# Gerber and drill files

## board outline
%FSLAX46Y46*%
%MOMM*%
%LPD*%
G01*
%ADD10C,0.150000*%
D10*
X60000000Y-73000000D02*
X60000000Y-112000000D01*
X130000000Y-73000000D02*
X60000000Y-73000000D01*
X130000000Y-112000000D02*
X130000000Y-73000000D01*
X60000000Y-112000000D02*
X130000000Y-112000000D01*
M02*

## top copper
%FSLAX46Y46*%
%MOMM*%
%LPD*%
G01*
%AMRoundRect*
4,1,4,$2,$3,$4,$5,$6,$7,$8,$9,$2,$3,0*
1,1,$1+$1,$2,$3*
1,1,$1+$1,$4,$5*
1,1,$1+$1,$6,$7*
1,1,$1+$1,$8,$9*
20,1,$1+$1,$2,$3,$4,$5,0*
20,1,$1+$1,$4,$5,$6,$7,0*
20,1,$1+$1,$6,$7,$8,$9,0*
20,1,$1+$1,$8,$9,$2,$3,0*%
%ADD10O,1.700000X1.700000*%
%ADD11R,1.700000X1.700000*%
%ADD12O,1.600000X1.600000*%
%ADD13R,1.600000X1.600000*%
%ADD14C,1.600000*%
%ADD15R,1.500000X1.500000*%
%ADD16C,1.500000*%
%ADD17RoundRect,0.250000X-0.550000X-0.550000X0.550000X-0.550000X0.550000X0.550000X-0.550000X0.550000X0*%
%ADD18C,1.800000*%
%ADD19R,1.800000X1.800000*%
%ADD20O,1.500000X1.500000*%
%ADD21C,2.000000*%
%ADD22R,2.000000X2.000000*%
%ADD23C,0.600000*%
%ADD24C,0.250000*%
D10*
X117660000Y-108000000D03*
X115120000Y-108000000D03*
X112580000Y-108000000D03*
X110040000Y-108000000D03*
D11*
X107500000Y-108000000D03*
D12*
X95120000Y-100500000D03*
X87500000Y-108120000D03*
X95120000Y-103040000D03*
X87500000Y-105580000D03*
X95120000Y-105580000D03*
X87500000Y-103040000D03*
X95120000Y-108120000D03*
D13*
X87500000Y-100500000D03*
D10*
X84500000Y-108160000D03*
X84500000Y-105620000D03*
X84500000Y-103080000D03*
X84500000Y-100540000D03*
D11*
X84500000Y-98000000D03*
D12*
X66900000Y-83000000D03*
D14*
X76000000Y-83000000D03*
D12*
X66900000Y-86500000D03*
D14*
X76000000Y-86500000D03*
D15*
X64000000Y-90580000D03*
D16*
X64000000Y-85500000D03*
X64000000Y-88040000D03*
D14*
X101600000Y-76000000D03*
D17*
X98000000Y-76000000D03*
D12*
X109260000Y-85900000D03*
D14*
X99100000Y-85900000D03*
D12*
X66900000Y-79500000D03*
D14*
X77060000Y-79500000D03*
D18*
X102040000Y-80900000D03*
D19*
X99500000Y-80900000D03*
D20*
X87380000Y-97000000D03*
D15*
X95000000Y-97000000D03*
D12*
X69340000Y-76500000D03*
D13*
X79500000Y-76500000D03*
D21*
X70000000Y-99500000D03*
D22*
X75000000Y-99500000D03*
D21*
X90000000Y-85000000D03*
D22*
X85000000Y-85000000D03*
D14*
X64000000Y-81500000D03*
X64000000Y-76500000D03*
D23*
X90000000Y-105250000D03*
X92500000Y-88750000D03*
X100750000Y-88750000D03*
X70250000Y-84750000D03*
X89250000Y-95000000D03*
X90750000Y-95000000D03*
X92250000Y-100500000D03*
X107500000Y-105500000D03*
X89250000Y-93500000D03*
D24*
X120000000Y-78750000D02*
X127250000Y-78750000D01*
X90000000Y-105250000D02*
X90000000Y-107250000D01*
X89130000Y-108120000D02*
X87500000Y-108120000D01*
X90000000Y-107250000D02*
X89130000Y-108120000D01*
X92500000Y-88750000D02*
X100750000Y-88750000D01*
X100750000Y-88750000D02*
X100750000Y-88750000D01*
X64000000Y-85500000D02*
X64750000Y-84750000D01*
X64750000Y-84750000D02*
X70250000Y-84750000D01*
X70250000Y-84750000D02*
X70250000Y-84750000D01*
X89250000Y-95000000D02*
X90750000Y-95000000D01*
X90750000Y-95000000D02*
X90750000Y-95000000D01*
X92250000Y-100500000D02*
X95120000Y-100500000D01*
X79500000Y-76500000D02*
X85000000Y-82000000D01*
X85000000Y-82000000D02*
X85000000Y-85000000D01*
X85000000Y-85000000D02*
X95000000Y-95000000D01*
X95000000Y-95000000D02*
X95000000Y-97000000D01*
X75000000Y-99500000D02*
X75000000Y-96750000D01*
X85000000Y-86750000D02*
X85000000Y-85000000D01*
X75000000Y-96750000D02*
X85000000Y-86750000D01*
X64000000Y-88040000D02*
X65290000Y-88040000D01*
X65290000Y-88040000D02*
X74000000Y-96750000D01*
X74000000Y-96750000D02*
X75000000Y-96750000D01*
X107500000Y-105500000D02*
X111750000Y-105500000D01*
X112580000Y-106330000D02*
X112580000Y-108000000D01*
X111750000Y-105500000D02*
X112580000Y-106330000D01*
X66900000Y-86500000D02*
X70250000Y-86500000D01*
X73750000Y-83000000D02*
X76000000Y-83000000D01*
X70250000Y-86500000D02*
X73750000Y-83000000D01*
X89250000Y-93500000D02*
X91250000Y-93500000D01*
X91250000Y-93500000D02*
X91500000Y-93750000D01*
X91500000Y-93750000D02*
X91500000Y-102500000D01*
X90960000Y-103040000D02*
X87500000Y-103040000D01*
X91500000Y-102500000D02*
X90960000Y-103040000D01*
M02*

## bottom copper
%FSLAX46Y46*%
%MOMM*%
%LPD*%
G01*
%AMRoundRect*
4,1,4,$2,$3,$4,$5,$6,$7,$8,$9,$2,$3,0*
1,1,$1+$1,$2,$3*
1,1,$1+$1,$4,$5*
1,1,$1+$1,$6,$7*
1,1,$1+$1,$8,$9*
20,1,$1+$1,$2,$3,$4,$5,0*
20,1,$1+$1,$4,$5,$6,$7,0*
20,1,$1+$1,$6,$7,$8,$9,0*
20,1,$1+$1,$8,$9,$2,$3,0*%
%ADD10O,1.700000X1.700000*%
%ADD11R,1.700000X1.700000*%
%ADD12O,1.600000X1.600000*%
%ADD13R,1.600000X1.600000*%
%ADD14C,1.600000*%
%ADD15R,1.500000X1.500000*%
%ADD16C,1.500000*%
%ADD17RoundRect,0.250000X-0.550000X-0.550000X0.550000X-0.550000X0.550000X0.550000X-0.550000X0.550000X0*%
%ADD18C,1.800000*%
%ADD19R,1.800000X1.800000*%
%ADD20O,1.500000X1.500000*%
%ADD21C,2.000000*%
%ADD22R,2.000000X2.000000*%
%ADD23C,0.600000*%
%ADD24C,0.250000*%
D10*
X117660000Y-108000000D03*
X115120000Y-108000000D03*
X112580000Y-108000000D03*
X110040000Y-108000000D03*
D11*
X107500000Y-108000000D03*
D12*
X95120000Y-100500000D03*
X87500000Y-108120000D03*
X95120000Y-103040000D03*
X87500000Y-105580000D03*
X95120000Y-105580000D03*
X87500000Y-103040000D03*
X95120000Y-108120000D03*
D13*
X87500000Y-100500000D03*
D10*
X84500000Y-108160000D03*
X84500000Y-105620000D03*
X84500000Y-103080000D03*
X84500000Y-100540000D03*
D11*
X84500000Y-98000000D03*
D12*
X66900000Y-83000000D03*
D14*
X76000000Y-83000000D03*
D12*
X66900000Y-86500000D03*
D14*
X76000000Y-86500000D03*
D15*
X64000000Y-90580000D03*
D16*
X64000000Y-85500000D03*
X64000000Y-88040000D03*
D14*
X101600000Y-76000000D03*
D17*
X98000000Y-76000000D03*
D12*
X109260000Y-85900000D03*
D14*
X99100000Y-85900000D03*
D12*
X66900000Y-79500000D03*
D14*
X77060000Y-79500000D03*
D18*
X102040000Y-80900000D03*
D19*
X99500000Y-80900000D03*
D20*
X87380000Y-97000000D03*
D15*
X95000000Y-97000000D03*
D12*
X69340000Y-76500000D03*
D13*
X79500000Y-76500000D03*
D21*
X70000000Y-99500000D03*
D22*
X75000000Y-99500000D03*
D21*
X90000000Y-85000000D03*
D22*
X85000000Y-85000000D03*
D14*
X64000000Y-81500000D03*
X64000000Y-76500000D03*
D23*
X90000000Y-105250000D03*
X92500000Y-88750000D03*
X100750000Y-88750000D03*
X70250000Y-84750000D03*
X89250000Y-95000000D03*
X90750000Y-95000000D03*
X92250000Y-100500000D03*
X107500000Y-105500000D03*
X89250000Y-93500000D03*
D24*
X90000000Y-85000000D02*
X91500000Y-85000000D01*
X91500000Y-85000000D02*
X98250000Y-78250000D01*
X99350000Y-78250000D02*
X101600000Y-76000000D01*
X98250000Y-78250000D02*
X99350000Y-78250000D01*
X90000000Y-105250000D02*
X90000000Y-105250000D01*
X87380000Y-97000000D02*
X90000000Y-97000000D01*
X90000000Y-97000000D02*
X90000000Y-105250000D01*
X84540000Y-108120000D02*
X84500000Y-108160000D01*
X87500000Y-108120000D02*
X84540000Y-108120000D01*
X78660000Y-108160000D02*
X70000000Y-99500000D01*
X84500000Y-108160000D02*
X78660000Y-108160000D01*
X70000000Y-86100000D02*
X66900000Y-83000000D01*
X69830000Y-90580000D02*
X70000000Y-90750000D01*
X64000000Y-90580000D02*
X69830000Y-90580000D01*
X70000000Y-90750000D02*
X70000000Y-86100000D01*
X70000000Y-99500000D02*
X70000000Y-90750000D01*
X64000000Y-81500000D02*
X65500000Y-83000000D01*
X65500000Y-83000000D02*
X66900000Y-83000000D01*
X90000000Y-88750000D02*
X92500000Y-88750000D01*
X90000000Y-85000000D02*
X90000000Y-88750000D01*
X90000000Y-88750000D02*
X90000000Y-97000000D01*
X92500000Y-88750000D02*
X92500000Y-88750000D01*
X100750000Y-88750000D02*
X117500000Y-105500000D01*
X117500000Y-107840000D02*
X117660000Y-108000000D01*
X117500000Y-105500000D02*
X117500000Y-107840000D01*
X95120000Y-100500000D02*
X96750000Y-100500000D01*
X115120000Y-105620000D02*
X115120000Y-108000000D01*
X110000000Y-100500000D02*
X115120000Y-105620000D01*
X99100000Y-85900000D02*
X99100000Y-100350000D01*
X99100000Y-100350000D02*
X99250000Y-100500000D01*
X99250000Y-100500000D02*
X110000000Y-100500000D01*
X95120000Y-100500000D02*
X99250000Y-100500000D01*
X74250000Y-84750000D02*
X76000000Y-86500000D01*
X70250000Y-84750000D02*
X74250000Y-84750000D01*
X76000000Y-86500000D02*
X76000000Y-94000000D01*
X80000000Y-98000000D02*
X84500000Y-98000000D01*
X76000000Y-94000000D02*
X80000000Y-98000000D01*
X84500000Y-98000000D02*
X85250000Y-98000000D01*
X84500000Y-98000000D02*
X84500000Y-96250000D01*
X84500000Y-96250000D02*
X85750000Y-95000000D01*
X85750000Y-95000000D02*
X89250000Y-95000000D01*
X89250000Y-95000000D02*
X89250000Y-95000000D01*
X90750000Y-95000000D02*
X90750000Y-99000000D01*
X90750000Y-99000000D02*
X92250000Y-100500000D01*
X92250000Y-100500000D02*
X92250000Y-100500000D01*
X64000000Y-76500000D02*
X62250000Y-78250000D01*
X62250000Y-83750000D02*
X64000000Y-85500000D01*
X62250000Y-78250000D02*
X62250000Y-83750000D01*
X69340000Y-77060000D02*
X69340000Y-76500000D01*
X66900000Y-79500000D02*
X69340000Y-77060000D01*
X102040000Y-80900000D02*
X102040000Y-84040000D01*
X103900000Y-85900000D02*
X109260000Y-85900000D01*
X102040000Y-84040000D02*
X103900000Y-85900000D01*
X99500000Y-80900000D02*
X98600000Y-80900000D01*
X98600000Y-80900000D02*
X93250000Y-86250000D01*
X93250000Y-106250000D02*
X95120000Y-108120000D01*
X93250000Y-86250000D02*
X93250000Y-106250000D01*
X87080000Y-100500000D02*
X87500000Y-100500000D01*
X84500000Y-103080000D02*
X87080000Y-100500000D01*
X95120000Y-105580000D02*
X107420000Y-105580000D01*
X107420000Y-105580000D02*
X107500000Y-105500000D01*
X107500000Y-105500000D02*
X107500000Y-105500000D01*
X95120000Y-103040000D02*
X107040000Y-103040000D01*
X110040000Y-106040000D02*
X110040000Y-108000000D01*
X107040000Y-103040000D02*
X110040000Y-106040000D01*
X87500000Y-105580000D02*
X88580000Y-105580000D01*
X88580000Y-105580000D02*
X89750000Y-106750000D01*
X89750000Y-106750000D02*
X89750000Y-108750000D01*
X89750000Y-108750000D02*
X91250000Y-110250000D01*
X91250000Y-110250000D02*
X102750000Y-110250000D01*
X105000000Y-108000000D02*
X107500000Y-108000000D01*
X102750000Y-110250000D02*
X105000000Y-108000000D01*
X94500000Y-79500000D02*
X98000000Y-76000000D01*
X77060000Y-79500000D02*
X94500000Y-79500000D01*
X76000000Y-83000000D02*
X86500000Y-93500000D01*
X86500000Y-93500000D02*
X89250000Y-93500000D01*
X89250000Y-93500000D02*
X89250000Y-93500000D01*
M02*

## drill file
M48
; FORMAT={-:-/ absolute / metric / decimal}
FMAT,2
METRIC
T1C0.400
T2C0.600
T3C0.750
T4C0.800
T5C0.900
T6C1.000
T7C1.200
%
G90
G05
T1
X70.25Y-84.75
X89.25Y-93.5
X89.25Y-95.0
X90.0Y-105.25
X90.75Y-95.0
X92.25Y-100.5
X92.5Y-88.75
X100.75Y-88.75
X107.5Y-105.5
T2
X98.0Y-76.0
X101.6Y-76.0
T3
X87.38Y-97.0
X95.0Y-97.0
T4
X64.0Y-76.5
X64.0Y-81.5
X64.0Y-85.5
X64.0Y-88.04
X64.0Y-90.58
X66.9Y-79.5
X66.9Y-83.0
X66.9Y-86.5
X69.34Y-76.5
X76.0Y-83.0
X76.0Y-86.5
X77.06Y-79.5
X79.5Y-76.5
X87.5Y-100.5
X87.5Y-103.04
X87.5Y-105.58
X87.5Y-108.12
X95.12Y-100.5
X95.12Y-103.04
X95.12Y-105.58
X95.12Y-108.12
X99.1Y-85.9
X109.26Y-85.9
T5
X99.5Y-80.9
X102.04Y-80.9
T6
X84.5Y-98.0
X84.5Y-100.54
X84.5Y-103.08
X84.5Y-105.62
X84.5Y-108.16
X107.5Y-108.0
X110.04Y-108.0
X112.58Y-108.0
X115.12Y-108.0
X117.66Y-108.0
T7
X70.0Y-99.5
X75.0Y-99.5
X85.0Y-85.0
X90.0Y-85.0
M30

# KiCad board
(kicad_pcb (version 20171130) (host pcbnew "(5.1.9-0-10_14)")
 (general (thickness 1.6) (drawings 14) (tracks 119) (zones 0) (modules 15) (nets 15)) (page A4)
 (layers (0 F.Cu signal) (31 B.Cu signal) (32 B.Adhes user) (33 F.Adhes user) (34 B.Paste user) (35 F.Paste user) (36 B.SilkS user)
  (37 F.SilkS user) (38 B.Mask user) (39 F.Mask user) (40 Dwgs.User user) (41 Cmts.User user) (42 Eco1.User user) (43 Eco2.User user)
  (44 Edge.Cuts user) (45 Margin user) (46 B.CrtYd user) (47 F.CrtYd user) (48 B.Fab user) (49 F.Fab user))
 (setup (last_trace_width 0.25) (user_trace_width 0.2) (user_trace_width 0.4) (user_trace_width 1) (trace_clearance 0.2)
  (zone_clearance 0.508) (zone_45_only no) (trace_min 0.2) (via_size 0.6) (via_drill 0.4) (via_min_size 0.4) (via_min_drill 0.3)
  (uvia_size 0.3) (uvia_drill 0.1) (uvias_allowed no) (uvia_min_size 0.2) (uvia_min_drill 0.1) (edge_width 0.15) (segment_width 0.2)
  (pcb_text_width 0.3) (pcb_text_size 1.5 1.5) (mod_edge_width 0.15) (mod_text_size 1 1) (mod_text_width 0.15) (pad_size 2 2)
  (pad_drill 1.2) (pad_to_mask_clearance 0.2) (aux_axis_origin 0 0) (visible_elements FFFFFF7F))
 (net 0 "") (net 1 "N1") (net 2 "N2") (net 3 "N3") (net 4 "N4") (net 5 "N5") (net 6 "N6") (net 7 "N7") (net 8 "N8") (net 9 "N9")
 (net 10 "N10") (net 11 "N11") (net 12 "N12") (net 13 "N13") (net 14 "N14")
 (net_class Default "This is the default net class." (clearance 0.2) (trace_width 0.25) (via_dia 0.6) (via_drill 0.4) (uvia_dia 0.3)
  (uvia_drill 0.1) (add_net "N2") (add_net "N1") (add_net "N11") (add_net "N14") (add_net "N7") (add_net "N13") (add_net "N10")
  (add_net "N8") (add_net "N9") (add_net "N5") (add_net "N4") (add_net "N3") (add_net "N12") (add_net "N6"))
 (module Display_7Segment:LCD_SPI (layer F.Cu) (at 97.5 110 90)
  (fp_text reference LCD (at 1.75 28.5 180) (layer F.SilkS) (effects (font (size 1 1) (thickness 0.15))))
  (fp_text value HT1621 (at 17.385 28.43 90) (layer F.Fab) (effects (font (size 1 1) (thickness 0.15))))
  (pad 5 thru_hole oval (at 2 20.16 90) (size 1.7 1.7) (drill 1) (layers *.Cu *.Mask) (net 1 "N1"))
  (pad 4 thru_hole oval (at 2 17.62 90) (size 1.7 1.7) (drill 1) (layers *.Cu *.Mask) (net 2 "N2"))
  (pad 3 thru_hole oval (at 2 15.08 90) (size 1.7 1.7) (drill 1) (layers *.Cu *.Mask) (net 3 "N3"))
  (pad 2 thru_hole oval (at 2 12.54 90) (size 1.7 1.7) (drill 1) (layers *.Cu *.Mask) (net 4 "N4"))
  (pad 1 thru_hole rect (at 2 10 90) (size 1.7 1.7) (drill 1) (layers *.Cu *.Mask) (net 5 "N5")))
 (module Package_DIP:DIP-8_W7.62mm (layer F.Cu) (at 87.5 100.5)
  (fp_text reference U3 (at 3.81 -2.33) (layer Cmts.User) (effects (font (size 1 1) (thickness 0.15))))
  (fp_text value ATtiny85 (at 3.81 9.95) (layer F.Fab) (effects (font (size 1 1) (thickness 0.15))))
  (pad 8 thru_hole oval (at 7.62 0) (size 1.6 1.6) (drill 0.8) (layers *.Cu *.Mask) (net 2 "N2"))
  (pad 4 thru_hole oval (at 0 7.62) (size 1.6 1.6) (drill 0.8) (layers *.Cu *.Mask) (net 1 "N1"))
  (pad 7 thru_hole oval (at 7.62 2.54) (size 1.6 1.6) (drill 0.8) (layers *.Cu *.Mask) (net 4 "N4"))
  (pad 3 thru_hole oval (at 0 5.08) (size 1.6 1.6) (drill 0.8) (layers *.Cu *.Mask) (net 5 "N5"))
  (pad 6 thru_hole oval (at 7.62 5.08) (size 1.6 1.6) (drill 0.8) (layers *.Cu *.Mask) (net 3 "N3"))
  (pad 2 thru_hole oval (at 0 2.54) (size 1.6 1.6) (drill 0.8) (layers *.Cu *.Mask) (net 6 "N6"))
  (pad 5 thru_hole oval (at 7.62 7.62) (size 1.6 1.6) (drill 0.8) (layers *.Cu *.Mask) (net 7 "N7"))
  (pad 1 thru_hole rect (at 0 0) (size 1.6 1.6) (drill 0.8) (layers *.Cu *.Mask) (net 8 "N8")))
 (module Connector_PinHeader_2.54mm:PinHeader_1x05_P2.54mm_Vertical (layer F.Cu) (at 84.5 98)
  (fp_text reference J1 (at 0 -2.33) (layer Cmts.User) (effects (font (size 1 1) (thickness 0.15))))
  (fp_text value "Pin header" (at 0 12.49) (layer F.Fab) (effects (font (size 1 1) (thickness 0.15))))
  (pad 5 thru_hole oval (at 0 10.16) (size 1.7 1.7) (drill 1) (layers *.Cu *.Mask) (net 1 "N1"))
  (pad 4 thru_hole oval (at 0 7.62) (size 1.7 1.7) (drill 1) (layers *.Cu *.Mask) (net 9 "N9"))
  (pad 3 thru_hole oval (at 0 5.08) (size 1.7 1.7) (drill 1) (layers *.Cu *.Mask) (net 8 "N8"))
  (pad 2 thru_hole oval (at 0 2.54) (size 1.7 1.7) (drill 1) (layers *.Cu *.Mask) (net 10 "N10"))
  (pad 1 thru_hole rect (at 0 0) (size 1.7 1.7) (drill 1) (layers *.Cu *.Mask) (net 2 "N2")))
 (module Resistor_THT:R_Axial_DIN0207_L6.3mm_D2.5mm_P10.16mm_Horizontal (layer F.Cu) (at 77 83 180)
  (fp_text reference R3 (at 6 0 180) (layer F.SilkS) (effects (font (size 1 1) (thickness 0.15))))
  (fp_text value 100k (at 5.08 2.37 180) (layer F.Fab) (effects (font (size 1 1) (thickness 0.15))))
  (pad 2 thru_hole oval (at 10.1 0 180) (size 1.6 1.6) (drill 0.8) (layers *.Cu *.Mask) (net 1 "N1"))
  (pad 1 thru_hole circle (at 1 0 180) (size 1.6 1.6) (drill 0.8) (layers *.Cu *.Mask) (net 6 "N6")))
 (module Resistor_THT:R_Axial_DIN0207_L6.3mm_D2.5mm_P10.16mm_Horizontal (layer F.Cu) (at 77 86.5 180)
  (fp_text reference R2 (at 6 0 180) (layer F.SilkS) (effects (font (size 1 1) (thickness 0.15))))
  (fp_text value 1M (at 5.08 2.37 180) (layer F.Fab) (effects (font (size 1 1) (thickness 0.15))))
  (pad 2 thru_hole oval (at 10.1 0 180) (size 1.6 1.6) (drill 0.8) (layers *.Cu *.Mask) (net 6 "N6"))
  (pad 1 thru_hole circle (at 1 0 180) (size 1.6 1.6) (drill 0.8) (layers *.Cu *.Mask) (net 2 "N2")))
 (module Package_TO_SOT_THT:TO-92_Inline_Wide (layer F.Cu) (at 64 90.58 90)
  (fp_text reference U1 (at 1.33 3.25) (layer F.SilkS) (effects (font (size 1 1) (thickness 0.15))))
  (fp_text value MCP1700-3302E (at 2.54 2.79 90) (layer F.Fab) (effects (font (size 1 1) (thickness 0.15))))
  (pad 1 thru_hole rect (at 0 0 90) (size 1.5 1.5) (drill 0.8) (layers *.Cu *.Mask) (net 1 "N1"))
  (pad 3 thru_hole circle (at 5.08 0 90) (size 1.5 1.5) (drill 0.8) (layers *.Cu *.Mask) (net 2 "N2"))
  (pad 2 thru_hole circle (at 2.54 0 90) (size 1.5 1.5) (drill 0.8) (layers *.Cu *.Mask) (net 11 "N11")))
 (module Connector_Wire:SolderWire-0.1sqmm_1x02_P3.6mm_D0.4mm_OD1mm (layer F.Cu) (at 98 76)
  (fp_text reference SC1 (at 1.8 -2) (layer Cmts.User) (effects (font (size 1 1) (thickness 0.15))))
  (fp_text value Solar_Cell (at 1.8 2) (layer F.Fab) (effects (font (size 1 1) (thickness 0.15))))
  (pad 2 thru_hole circle (at 3.6 0) (size 1.6 1.6) (drill 0.6) (layers *.Cu *.Mask) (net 1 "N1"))
  (pad 1 thru_hole roundrect (at 0 0) (size 1.6 1.6) (drill 0.6) (layers *.Cu *.Mask) (roundrect_rratio 0.15625) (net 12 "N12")))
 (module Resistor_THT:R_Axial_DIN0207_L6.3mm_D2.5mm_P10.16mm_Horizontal (layer F.Cu) (at 99.1 85.9)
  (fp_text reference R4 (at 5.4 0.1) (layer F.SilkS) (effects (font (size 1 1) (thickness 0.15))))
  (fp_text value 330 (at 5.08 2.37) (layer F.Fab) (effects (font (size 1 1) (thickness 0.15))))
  (pad 2 thru_hole oval (at 10.16 0) (size 1.6 1.6) (drill 0.8) (layers *.Cu *.Mask) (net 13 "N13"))
  (pad 1 thru_hole circle (at 0 0) (size 1.6 1.6) (drill 0.8) (layers *.Cu *.Mask) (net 2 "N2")))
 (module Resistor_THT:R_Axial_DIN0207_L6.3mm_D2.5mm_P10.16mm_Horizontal (layer F.Cu) (at 77.06 79.5 180)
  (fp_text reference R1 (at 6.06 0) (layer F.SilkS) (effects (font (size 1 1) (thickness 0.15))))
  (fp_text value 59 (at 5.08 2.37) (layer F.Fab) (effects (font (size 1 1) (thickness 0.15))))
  (pad 2 thru_hole oval (at 10.16 0 180) (size 1.6 1.6) (drill 0.8) (layers *.Cu *.Mask) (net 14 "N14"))
  (pad 1 thru_hole circle (at 0 0 180) (size 1.6 1.6) (drill 0.8) (layers *.Cu *.Mask) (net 12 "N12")))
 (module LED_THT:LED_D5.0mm (layer F.Cu) (at 99.5 80.9)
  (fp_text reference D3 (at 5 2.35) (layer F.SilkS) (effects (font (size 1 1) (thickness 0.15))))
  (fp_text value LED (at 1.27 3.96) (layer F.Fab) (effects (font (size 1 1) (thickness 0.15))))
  (pad 2 thru_hole circle (at 2.54 0) (size 1.8 1.8) (drill 0.9) (layers *.Cu *.Mask) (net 13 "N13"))
  (pad 1 thru_hole rect (at 0 0) (size 1.8 1.8) (drill 0.9) (layers *.Cu *.Mask) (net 7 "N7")))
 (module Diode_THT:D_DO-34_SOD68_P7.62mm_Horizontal (layer F.Cu) (at 95 97 180)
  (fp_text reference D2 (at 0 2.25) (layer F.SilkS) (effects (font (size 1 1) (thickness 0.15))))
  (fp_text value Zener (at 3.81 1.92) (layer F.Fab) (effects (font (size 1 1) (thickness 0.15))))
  (pad 2 thru_hole oval (at 7.62 0 180) (size 1.5 1.5) (drill 0.75) (layers *.Cu *.Mask) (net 1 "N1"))
  (pad 1 thru_hole rect (at 0 0 180) (size 1.5 1.5) (drill 0.75) (layers *.Cu *.Mask) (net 11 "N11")))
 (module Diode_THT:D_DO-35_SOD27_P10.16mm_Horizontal (layer F.Cu) (at 79.5 76.5 180)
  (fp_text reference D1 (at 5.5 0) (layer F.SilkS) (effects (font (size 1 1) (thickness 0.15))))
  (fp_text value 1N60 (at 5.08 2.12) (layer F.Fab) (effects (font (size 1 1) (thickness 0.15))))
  (pad 2 thru_hole oval (at 10.16 0 180) (size 1.6 1.6) (drill 0.8) (layers *.Cu *.Mask) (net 14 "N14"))
  (pad 1 thru_hole rect (at 0 0 180) (size 1.6 1.6) (drill 0.8) (layers *.Cu *.Mask) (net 11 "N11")))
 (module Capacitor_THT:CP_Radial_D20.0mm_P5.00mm (layer F.Cu) (at 75 99.5 180)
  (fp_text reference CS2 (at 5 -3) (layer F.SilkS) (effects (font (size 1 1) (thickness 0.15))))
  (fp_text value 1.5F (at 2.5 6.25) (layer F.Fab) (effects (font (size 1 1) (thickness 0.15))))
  (pad 2 thru_hole circle (at 5 0 180) (size 2 2) (drill 1.2) (layers *.Cu *.Mask) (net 1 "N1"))
  (pad 1 thru_hole rect (at 0 0 180) (size 2 2) (drill 1.2) (layers *.Cu *.Mask) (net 11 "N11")))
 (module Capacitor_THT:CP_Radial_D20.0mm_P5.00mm (layer F.Cu) (at 85 85)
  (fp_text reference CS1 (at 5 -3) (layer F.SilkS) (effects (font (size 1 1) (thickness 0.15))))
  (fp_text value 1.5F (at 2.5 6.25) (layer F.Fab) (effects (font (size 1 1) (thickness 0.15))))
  (pad 2 thru_hole circle (at 5 0) (size 2 2) (drill 1.2) (layers *.Cu *.Mask) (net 1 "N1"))
  (pad 1 thru_hole rect (at 0 0) (size 2 2) (drill 1.2) (layers *.Cu *.Mask) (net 11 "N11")))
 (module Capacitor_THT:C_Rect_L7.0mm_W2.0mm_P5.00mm (layer F.Cu) (at 64 76.5 270)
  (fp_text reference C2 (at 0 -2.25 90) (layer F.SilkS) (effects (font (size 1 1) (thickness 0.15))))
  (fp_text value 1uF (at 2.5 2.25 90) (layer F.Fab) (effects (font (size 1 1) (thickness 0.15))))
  (pad 2 thru_hole circle (at 5 0 270) (size 1.6 1.6) (drill 0.8) (layers *.Cu *.Mask) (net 1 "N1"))
  (pad 1 thru_hole circle (at 0 0 270) (size 1.6 1.6) (drill 0.8) (layers *.Cu *.Mask) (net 2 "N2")))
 (gr_line (start 60 73) (end 60 112) (layer Edge.Cuts) (width 0.15))
 (gr_line (start 130 73) (end 60 73) (layer Edge.Cuts) (width 0.15))
 (gr_line (start 130 112) (end 130 73) (layer Edge.Cuts) (width 0.15))
 (gr_line (start 60 112) (end 130 112) (layer Edge.Cuts) (width 0.15))
 (segment (start 120 78.75) (end 127.25 78.75) (width 0.25) (layer F.Cu) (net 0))
 (segment (start 90 85) (end 91.5 85) (width 0.25) (layer B.Cu) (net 1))
 (segment (start 91.5 85) (end 98.25 78.25) (width 0.25) (layer B.Cu) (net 1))
 (segment (start 99.35 78.25) (end 101.6 76) (width 0.25) (layer B.Cu) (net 1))
 (segment (start 98.25 78.25) (end 99.35 78.25) (width 0.25) (layer B.Cu) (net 1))
 (segment (start 90 105.25) (end 90 105.25) (width 0.25) (layer B.Cu) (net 1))
 (via (at 90 105.25) (size 0.6) (drill 0.4) (layers F.Cu B.Cu) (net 1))
 (segment (start 90 105.25) (end 90 107.25) (width 0.25) (layer F.Cu) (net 1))
 (segment (start 89.13 108.12) (end 87.5 108.12) (width 0.25) (layer F.Cu) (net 1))
 (segment (start 90 107.25) (end 89.13 108.12) (width 0.25) (layer F.Cu) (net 1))
 (segment (start 87.38 97) (end 90 97) (width 0.25) (layer B.Cu) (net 1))
 (segment (start 90 97) (end 90 105.25) (width 0.25) (layer B.Cu) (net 1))
 (segment (start 84.54 108.12) (end 84.5 108.16) (width 0.25) (layer B.Cu) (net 1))
 (segment (start 87.5 108.12) (end 84.54 108.12) (width 0.25) (layer B.Cu) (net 1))
 (segment (start 78.66 108.16) (end 70 99.5) (width 0.25) (layer B.Cu) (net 1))
 (segment (start 84.5 108.16) (end 78.66 108.16) (width 0.25) (layer B.Cu) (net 1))
 (segment (start 70 86.1) (end 66.9 83) (width 0.25) (layer B.Cu) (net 1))
 (segment (start 69.83 90.58) (end 70 90.75) (width 0.25) (layer B.Cu) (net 1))
 (segment (start 64 90.58) (end 69.83 90.58) (width 0.25) (layer B.Cu) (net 1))
 (segment (start 70 90.75) (end 70 86.1) (width 0.25) (layer B.Cu) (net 1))
 (segment (start 70 99.5) (end 70 90.75) (width 0.25) (layer B.Cu) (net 1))
 (segment (start 64 81.5) (end 65.5 83) (width 0.25) (layer B.Cu) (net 1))
 (segment (start 65.5 83) (end 66.9 83) (width 0.25) (layer B.Cu) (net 1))
 (segment (start 90 88.75) (end 92.5 88.75) (width 0.25) (layer B.Cu) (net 1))
 (segment (start 90 85) (end 90 88.75) (width 0.25) (layer B.Cu) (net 1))
 (segment (start 90 88.75) (end 90 97) (width 0.25) (layer B.Cu) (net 1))
 (segment (start 92.5 88.75) (end 92.5 88.75) (width 0.25) (layer B.Cu) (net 1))
 (via (at 92.5 88.75) (size 0.6) (drill 0.4) (layers F.Cu B.Cu) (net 1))
 (segment (start 92.5 88.75) (end 100.75 88.75) (width 0.25) (layer F.Cu) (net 1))
 (segment (start 100.75 88.75) (end 100.75 88.75) (width 0.25) (layer F.Cu) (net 1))
 (via (at 100.75 88.75) (size 0.6) (drill 0.4) (layers F.Cu B.Cu) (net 1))
 (segment (start 100.75 88.75) (end 117.5 105.5) (width 0.25) (layer B.Cu) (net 1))
 (segment (start 117.5 107.84) (end 117.66 108) (width 0.25) (layer B.Cu) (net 1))
 (segment (start 117.5 105.5) (end 117.5 107.84) (width 0.25) (layer B.Cu) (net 1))
 (segment (start 95.12 100.5) (end 96.75 100.5) (width 0.25) (layer B.Cu) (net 2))
 (segment (start 115.12 105.62) (end 115.12 108) (width 0.25) (layer B.Cu) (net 2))
 (segment (start 110 100.5) (end 115.12 105.62) (width 0.25) (layer B.Cu) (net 2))
 (segment (start 99.1 85.9) (end 99.1 100.35) (width 0.25) (layer B.Cu) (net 2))
 (segment (start 99.1 100.35) (end 99.25 100.5) (width 0.25) (layer B.Cu) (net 2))
 (segment (start 99.25 100.5) (end 110 100.5) (width 0.25) (layer B.Cu) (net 2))
 (segment (start 95.12 100.5) (end 99.25 100.5) (width 0.25) (layer B.Cu) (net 2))
 (segment (start 64 85.5) (end 64.75 84.75) (width 0.25) (layer F.Cu) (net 2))
 (segment (start 64.75 84.75) (end 70.25 84.75) (width 0.25) (layer F.Cu) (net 2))
 (segment (start 70.25 84.75) (end 70.25 84.75) (width 0.25) (layer F.Cu) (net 2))
 (via (at 70.25 84.75) (size 0.6) (drill 0.4) (layers F.Cu B.Cu) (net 2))
 (segment (start 74.25 84.75) (end 76 86.5) (width 0.25) (layer B.Cu) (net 2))
 (segment (start 70.25 84.75) (end 74.25 84.75) (width 0.25) (layer B.Cu) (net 2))
 (segment (start 76 86.5) (end 76 94) (width 0.25) (layer B.Cu) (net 2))
 (segment (start 80 98) (end 84.5 98) (width 0.25) (layer B.Cu) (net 2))
 (segment (start 76 94) (end 80 98) (width 0.25) (layer B.Cu) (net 2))
 (segment (start 84.5 98) (end 85.25 98) (width 0.25) (layer B.Cu) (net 2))
 (segment (start 84.5 98) (end 84.5 96.25) (width 0.25) (layer B.Cu) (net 2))
 (segment (start 84.5 96.25) (end 85.75 95) (width 0.25) (layer B.Cu) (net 2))
 (segment (start 85.75 95) (end 89.25 95) (width 0.25) (layer B.Cu) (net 2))
 (segment (start 89.25 95) (end 89.25 95) (width 0.25) (layer B.Cu) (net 2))
 (via (at 89.25 95) (size 0.6) (drill 0.4) (layers F.Cu B.Cu) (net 2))
 (segment (start 89.25 95) (end 90.75 95) (width 0.25) (layer F.Cu) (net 2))
 (segment (start 90.75 95) (end 90.75 95) (width 0.25) (layer F.Cu) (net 2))
 (via (at 90.75 95) (size 0.6) (drill 0.4) (layers F.Cu B.Cu) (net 2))
 (segment (start 90.75 95) (end 90.75 99) (width 0.25) (layer B.Cu) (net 2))
 (segment (start 90.75 99) (end 92.25 100.5) (width 0.25) (layer B.Cu) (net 2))
 (segment (start 92.25 100.5) (end 92.25 100.5) (width 0.25) (layer B.Cu) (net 2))
 (via (at 92.25 100.5) (size 0.6) (drill 0.4) (layers F.Cu B.Cu) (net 2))
 (segment (start 92.25 100.5) (end 95.12 100.5) (width 0.25) (layer F.Cu) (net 2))
 (segment (start 64 76.5) (end 62.25 78.25) (width 0.25) (layer B.Cu) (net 2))
 (segment (start 62.25 83.75) (end 64 85.5) (width 0.25) (layer B.Cu) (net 2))
 (segment (start 62.25 78.25) (end 62.25 83.75) (width 0.25) (layer B.Cu) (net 2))
 (segment (start 79.5 76.5) (end 85 82) (width 0.25) (layer F.Cu) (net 11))
 (segment (start 85 82) (end 85 85) (width 0.25) (layer F.Cu) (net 11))
 (segment (start 85 85) (end 95 95) (width 0.25) (layer F.Cu) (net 11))
 (segment (start 95 95) (end 95 97) (width 0.25) (layer F.Cu) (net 11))
 (segment (start 75 99.5) (end 75 96.75) (width 0.25) (layer F.Cu) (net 11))
 (segment (start 85 86.75) (end 85 85) (width 0.25) (layer F.Cu) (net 11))
 (segment (start 75 96.75) (end 85 86.75) (width 0.25) (layer F.Cu) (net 11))
 (segment (start 64 88.04) (end 65.29 88.04) (width 0.25) (layer F.Cu) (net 11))
 (segment (start 65.29 88.04) (end 74 96.75) (width 0.25) (layer F.Cu) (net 11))
 (segment (start 74 96.75) (end 75 96.75) (width 0.25) (layer F.Cu) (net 11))
 (segment (start 69.34 77.06) (end 69.34 76.5) (width 0.25) (layer B.Cu) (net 14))
 (segment (start 66.9 79.5) (end 69.34 77.06) (width 0.25) (layer B.Cu) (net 14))
 (segment (start 102.04 80.9) (end 102.04 84.04) (width 0.25) (layer B.Cu) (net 13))
 (segment (start 103.9 85.9) (end 109.26 85.9) (width 0.25) (layer B.Cu) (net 13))
 (segment (start 102.04 84.04) (end 103.9 85.9) (width 0.25) (layer B.Cu) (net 13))
 (segment (start 99.5 80.9) (end 98.6 80.9) (width 0.25) (layer B.Cu) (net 7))
 (segment (start 98.6 80.9) (end 93.25 86.25) (width 0.25) (layer B.Cu) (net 7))
 (segment (start 93.25 106.25) (end 95.12 108.12) (width 0.25) (layer B.Cu) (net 7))
 (segment (start 93.25 86.25) (end 93.25 106.25) (width 0.25) (layer B.Cu) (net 7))
 (segment (start 87.08 100.5) (end 87.5 100.5) (width 0.25) (layer B.Cu) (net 8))
 (segment (start 84.5 103.08) (end 87.08 100.5) (width 0.25) (layer B.Cu) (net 8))
 (segment (start 95.12 105.58) (end 107.42 105.58) (width 0.25) (layer B.Cu) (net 3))
 (segment (start 107.42 105.58) (end 107.5 105.5) (width 0.25) (layer B.Cu) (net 3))
 (segment (start 107.5 105.5) (end 107.5 105.5) (width 0.25) (layer B.Cu) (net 3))
 (via (at 107.5 105.5) (size 0.6) (drill 0.4) (layers F.Cu B.Cu) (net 3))
 (segment (start 107.5 105.5) (end 111.75 105.5) (width 0.25) (layer F.Cu) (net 3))
 (segment (start 112.58 106.33) (end 112.58 108) (width 0.25) (layer F.Cu) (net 3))
 (segment (start 111.75 105.5) (end 112.58 106.33) (width 0.25) (layer F.Cu) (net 3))
 (segment (start 95.12 103.04) (end 107.04 103.04) (width 0.25) (layer B.Cu) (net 4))
 (segment (start 110.04 106.04) (end 110.04 108) (width 0.25) (layer B.Cu) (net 4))
 (segment (start 107.04 103.04) (end 110.04 106.04) (width 0.25) (layer B.Cu) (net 4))
 (segment (start 87.5 105.58) (end 88.58 105.58) (width 0.25) (layer B.Cu) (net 5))
 (segment (start 88.58 105.58) (end 89.75 106.75) (width 0.25) (layer B.Cu) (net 5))
 (segment (start 89.75 106.75) (end 89.75 108.75) (width 0.25) (layer B.Cu) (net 5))
 (segment (start 89.75 108.75) (end 91.25 110.25) (width 0.25) (layer B.Cu) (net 5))
 (segment (start 91.25 110.25) (end 102.75 110.25) (width 0.25) (layer B.Cu) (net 5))
 (segment (start 105 108) (end 107.5 108) (width 0.25) (layer B.Cu) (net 5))
 (segment (start 102.75 110.25) (end 105 108) (width 0.25) (layer B.Cu) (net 5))
 (segment (start 94.5 79.5) (end 98 76) (width 0.25) (layer B.Cu) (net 12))
 (segment (start 77.06 79.5) (end 94.5 79.5) (width 0.25) (layer B.Cu) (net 12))
 (segment (start 66.9 86.5) (end 70.25 86.5) (width 0.25) (layer F.Cu) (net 6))
 (segment (start 73.75 83) (end 76 83) (width 0.25) (layer F.Cu) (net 6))
 (segment (start 70.25 86.5) (end 73.75 83) (width 0.25) (layer F.Cu) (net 6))
 (segment (start 76 83) (end 86.5 93.5) (width 0.25) (layer B.Cu) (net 6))
 (segment (start 86.5 93.5) (end 89.25 93.5) (width 0.25) (layer B.Cu) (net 6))
 (segment (start 89.25 93.5) (end 89.25 93.5) (width 0.25) (layer B.Cu) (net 6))
 (via (at 89.25 93.5) (size 0.6) (drill 0.4) (layers F.Cu B.Cu) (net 6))
 (segment (start 89.25 93.5) (end 91.25 93.5) (width 0.25) (layer F.Cu) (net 6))
 (segment (start 91.25 93.5) (end 91.5 93.75) (width 0.25) (layer F.Cu) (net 6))
 (segment (start 91.5 93.75) (end 91.5 102.5) (width 0.25) (layer F.Cu) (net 6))
 (segment (start 90.96 103.04) (end 87.5 103.04) (width 0.25) (layer F.Cu) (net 6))
 (segment (start 91.5 102.5) (end 90.96 103.04) (width 0.25) (layer F.Cu) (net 6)))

